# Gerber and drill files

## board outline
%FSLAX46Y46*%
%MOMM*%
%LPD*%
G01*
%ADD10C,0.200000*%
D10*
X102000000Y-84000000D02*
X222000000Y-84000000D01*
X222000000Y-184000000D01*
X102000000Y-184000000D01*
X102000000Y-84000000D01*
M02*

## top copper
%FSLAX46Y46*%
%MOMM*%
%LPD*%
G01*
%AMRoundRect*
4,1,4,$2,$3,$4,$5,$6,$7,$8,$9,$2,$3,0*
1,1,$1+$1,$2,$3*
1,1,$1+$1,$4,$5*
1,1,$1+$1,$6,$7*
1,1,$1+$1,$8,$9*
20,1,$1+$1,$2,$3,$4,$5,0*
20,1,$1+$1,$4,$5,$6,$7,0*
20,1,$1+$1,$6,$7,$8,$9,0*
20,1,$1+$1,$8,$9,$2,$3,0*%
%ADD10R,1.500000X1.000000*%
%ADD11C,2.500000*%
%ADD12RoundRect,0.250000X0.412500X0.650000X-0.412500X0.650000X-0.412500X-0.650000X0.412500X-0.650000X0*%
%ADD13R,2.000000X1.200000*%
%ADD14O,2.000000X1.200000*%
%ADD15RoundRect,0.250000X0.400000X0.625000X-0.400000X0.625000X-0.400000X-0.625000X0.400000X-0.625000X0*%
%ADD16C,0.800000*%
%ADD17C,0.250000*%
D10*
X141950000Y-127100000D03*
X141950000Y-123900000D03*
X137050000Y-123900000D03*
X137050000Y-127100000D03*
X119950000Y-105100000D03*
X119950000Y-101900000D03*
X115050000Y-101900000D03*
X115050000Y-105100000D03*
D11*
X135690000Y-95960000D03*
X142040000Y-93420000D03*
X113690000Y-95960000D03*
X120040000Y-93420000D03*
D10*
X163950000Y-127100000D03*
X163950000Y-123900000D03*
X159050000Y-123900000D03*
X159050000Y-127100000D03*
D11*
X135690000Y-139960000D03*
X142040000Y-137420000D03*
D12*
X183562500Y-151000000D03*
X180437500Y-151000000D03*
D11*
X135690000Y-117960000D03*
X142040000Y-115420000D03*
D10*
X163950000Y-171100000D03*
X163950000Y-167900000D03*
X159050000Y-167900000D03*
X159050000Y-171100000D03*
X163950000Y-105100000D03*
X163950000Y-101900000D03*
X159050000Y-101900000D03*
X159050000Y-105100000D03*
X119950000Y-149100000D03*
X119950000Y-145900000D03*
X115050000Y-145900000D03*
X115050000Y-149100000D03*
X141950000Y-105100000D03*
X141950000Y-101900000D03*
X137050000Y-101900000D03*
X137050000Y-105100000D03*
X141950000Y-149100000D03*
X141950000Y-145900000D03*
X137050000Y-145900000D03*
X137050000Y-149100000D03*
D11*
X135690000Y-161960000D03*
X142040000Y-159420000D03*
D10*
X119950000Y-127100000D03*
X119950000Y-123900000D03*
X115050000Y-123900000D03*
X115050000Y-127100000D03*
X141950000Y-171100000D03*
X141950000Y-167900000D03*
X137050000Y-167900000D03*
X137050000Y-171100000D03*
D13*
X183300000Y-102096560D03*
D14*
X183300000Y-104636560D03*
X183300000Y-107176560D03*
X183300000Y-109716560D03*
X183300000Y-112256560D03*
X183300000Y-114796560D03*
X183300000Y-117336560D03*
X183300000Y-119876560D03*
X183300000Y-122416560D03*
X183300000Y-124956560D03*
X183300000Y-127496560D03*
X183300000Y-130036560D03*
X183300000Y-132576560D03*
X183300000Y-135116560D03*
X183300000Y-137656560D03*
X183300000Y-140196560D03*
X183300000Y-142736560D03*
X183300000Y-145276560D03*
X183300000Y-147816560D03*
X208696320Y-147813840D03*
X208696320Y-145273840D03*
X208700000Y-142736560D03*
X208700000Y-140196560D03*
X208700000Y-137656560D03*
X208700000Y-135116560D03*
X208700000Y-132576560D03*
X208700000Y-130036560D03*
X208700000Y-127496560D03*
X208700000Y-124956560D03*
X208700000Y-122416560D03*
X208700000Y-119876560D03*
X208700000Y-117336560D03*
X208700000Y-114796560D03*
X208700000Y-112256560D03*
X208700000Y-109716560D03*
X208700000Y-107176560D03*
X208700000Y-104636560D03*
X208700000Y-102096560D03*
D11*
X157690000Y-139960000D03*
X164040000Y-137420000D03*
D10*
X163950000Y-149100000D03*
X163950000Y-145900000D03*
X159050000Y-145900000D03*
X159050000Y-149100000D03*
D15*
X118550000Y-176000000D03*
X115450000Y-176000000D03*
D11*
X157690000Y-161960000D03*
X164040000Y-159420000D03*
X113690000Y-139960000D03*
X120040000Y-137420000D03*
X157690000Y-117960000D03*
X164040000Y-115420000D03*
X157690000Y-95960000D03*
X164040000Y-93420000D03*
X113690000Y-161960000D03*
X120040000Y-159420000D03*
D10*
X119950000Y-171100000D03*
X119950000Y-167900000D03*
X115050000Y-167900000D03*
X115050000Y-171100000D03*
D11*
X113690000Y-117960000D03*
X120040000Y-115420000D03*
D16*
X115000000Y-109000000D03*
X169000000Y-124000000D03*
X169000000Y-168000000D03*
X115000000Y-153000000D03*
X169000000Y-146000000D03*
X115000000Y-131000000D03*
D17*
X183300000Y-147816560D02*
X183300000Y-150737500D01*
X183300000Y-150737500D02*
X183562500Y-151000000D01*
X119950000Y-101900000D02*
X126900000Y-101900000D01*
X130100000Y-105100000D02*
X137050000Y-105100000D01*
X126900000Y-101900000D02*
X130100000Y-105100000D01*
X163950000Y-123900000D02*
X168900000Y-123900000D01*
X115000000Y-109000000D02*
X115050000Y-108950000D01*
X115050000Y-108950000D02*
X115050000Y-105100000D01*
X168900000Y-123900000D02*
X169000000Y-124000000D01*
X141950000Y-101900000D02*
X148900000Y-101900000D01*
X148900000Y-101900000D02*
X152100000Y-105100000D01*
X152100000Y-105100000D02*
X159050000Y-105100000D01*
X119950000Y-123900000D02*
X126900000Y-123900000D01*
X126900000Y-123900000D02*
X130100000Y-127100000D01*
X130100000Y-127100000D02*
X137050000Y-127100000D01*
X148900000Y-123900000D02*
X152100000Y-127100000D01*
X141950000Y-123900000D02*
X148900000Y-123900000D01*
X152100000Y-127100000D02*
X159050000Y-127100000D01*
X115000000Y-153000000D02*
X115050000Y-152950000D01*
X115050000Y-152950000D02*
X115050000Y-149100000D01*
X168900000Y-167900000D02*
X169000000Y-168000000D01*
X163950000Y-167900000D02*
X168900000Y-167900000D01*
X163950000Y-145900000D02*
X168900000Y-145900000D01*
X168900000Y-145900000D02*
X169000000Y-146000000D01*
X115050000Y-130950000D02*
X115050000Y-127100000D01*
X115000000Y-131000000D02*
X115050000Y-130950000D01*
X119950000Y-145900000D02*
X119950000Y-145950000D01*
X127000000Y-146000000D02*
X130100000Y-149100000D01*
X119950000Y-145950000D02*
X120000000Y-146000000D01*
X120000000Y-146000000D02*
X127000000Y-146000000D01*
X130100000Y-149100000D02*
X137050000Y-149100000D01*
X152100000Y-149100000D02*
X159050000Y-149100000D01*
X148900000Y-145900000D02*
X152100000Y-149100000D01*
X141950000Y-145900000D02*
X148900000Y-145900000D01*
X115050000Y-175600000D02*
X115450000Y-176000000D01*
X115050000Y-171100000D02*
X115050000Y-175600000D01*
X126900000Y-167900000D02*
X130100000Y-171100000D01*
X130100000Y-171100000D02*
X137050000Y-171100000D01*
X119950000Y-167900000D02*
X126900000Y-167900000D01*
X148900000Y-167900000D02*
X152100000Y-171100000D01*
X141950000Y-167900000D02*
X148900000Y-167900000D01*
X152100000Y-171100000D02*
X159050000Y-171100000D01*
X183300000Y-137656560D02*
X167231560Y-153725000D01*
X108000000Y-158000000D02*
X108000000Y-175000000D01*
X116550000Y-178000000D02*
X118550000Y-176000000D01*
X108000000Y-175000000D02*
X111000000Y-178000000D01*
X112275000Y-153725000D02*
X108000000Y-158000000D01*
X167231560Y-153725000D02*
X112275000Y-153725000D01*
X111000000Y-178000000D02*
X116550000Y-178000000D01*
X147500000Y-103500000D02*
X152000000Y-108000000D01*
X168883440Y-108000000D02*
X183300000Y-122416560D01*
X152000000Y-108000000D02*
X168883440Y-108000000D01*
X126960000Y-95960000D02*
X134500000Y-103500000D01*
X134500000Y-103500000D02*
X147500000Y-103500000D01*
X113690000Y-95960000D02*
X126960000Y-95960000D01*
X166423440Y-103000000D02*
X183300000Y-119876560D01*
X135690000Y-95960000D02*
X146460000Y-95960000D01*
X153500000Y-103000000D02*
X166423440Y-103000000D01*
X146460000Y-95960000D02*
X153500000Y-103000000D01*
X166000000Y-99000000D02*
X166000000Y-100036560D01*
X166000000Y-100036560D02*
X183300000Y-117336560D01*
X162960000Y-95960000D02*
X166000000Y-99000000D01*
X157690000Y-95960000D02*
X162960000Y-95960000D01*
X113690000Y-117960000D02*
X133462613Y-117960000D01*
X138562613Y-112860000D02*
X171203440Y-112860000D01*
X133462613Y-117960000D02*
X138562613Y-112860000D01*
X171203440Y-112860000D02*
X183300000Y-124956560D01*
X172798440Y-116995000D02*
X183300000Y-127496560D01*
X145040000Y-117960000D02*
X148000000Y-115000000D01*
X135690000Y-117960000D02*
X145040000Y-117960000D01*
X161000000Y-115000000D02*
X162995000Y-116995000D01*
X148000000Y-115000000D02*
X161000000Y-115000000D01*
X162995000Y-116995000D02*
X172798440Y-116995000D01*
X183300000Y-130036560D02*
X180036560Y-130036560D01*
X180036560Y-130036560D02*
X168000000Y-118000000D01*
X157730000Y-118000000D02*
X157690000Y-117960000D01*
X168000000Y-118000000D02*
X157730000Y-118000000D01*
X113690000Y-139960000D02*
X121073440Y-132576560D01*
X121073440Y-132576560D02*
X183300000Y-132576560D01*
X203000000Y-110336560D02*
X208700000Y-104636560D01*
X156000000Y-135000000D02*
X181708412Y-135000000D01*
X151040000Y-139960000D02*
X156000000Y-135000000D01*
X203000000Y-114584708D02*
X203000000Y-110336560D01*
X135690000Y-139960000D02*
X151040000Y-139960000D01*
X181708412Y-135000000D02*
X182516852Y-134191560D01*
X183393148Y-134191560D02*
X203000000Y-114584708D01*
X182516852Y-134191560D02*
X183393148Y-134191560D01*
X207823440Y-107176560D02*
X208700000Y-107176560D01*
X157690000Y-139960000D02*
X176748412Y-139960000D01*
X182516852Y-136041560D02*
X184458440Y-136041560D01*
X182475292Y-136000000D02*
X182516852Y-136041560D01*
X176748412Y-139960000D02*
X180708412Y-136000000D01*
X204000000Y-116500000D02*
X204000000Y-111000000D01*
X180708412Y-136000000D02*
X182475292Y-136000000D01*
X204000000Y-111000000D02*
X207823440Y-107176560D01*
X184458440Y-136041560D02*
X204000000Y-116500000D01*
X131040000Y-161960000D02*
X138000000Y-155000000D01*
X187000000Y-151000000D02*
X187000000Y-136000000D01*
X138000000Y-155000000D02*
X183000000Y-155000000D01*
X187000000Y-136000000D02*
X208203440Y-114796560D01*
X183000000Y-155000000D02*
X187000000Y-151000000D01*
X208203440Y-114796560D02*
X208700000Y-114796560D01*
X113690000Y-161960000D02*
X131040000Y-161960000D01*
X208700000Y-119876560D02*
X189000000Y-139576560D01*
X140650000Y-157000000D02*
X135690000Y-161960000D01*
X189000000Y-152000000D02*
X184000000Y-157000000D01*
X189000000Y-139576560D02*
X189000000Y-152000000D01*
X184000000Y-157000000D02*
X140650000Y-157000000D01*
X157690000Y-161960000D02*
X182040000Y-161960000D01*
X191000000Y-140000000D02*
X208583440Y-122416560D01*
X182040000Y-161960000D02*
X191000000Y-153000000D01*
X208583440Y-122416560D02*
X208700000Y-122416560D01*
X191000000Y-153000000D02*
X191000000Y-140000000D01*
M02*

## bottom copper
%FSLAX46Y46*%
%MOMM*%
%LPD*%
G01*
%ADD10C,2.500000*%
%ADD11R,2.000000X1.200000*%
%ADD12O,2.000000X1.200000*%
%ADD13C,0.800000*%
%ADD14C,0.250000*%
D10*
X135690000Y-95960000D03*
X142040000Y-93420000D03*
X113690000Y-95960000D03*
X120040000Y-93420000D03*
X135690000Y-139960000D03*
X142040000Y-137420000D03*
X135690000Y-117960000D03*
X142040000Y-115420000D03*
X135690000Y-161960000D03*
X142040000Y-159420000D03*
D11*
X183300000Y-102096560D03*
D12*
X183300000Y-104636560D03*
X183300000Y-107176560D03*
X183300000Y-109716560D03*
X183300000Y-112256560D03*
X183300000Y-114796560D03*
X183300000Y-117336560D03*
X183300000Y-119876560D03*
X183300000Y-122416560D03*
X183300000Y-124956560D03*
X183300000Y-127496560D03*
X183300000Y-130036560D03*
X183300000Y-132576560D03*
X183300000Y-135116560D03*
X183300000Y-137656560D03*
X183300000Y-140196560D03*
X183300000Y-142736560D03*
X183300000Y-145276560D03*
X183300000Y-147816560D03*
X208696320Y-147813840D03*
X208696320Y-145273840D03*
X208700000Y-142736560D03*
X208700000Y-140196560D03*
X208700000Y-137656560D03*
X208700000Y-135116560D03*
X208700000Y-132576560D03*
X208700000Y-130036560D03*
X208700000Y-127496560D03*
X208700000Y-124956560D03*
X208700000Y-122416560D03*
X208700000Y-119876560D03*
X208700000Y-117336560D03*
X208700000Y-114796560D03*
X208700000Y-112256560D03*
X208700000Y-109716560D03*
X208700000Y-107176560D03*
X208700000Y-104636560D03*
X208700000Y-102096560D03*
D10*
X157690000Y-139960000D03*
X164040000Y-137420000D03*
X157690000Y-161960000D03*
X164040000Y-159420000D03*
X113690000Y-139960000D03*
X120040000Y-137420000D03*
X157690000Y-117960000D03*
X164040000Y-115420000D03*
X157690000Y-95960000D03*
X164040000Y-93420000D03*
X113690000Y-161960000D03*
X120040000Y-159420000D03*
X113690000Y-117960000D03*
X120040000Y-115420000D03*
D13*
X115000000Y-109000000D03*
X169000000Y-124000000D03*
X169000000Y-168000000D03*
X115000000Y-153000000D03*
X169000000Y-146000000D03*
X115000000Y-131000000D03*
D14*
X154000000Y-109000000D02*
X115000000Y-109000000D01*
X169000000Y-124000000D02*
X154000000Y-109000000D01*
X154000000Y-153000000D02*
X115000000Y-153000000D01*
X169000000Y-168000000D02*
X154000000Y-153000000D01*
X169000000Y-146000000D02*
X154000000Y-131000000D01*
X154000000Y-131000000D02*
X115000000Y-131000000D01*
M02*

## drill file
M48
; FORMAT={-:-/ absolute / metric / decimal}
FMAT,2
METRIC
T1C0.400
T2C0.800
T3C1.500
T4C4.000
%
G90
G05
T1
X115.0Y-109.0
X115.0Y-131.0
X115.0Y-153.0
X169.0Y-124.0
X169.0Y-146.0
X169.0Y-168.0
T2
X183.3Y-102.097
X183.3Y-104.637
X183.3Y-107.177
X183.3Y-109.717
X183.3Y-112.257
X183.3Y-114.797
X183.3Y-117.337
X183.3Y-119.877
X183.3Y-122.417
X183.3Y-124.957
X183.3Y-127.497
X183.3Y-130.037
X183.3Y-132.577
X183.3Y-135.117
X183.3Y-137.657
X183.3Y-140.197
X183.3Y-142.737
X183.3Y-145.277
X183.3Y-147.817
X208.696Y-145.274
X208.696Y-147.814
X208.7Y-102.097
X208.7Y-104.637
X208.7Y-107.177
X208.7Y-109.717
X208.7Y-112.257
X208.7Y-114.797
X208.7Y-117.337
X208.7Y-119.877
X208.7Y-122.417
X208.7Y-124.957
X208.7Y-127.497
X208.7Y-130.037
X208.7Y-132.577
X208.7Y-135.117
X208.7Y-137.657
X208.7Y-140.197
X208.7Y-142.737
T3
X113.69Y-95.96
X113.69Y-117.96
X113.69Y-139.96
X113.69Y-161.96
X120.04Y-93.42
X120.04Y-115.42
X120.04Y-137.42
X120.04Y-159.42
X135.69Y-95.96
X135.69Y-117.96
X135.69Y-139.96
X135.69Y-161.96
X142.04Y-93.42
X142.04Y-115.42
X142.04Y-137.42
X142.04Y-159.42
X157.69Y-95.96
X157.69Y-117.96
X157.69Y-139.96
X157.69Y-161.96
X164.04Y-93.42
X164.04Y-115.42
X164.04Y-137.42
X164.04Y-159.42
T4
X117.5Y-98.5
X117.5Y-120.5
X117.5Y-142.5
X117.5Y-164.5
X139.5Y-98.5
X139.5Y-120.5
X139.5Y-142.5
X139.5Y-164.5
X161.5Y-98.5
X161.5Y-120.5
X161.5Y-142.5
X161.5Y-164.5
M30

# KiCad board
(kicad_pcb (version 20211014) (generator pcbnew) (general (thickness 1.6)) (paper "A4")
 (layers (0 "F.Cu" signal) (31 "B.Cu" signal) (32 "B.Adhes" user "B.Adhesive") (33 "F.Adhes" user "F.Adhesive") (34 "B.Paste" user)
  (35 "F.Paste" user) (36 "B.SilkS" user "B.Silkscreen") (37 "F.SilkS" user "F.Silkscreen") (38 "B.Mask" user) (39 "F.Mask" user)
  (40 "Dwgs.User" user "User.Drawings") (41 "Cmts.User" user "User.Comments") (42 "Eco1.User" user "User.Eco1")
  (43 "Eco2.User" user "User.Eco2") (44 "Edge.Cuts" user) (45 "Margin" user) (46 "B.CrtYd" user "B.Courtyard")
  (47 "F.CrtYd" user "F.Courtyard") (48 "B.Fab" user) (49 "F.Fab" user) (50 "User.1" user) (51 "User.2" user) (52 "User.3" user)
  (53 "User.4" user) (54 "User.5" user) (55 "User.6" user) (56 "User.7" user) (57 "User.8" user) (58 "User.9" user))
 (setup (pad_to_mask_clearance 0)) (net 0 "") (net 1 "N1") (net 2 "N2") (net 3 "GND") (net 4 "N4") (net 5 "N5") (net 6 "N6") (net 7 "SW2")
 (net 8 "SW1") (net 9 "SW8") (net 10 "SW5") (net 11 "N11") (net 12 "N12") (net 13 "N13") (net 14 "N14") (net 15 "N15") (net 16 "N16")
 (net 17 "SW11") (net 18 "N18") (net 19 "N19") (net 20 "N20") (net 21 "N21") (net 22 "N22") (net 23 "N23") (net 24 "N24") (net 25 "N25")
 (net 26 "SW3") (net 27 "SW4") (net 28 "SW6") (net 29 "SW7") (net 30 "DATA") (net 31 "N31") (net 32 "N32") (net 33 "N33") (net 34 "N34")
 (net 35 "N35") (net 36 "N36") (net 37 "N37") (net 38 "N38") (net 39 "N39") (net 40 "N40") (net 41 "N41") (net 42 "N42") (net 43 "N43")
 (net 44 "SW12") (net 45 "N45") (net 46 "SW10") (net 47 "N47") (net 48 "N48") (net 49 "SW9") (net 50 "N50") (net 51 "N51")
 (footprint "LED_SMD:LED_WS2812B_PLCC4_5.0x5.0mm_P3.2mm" (layer "F.Cu") (at 139.5 125.5 180)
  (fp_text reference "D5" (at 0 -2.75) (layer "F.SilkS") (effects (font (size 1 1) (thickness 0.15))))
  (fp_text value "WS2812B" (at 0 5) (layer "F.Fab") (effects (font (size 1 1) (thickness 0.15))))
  (pad "1" smd rect (at -2.45 -1.6 180) (size 1.5 1) (layers "F.Cu" "F.Paste" "F.Mask") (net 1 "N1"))
  (pad "2" smd rect (at -2.45 1.6 180) (size 1.5 1) (layers "F.Cu" "F.Paste" "F.Mask") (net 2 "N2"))
  (pad "3" smd rect (at 2.45 1.6 180) (size 1.5 1) (layers "F.Cu" "F.Paste" "F.Mask") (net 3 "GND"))
  (pad "4" smd rect (at 2.45 -1.6 180) (size 1.5 1) (layers "F.Cu" "F.Paste" "F.Mask") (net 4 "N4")))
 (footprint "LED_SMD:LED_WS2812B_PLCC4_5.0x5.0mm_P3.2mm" (layer "F.Cu") (at 117.5 103.5 180)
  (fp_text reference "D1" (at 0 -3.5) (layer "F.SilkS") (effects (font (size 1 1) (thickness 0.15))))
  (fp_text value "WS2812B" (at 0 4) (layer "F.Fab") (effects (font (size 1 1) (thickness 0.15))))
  (pad "1" smd rect (at -2.45 -1.6 180) (size 1.5 1) (layers "F.Cu" "F.Paste" "F.Mask") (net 1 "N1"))
  (pad "2" smd rect (at -2.45 1.6 180) (size 1.5 1) (layers "F.Cu" "F.Paste" "F.Mask") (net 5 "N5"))
  (pad "3" smd rect (at 2.45 1.6 180) (size 1.5 1) (layers "F.Cu" "F.Paste" "F.Mask") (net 3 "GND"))
  (pad "4" smd rect (at 2.45 -1.6 180) (size 1.5 1) (layers "F.Cu" "F.Paste" "F.Mask") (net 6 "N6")))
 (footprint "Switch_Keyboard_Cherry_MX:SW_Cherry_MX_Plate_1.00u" (layer "F.Cu") (at 139.5 98.5)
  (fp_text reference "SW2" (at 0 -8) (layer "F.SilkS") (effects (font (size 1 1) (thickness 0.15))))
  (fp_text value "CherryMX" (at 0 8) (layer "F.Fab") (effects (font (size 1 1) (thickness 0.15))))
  (pad "" np_thru_hole circle locked (at 0 0) (size 4 4) (drill 4) (layers *.Cu *.Mask))
  (pad "" smd circle locked (at -3.81 -2.54) (size 1.55 1.55) (layers "F.Mask"))
  (pad "" smd circle locked (at 2.54 -5.08) (size 1.55 1.55) (layers "F.Mask"))
  (pad "1" thru_hole circle locked (at -3.81 -2.54) (size 2.5 2.5) (drill 1.5) (layers *.Cu "B.Mask") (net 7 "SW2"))
  (pad "2" thru_hole circle locked (at 2.54 -5.08) (size 2.5 2.5) (drill 1.5) (layers *.Cu "B.Mask") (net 3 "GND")))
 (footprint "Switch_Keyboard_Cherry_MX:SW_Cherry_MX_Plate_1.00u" (layer "F.Cu") (at 117.5 98.5)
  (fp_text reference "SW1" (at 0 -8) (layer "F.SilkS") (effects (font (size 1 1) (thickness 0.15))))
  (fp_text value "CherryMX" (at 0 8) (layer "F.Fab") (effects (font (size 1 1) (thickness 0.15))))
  (pad "" smd circle locked (at -3.81 -2.54) (size 1.55 1.55) (layers "F.Mask"))
  (pad "" smd circle locked (at 2.54 -5.08) (size 1.55 1.55) (layers "F.Mask"))
  (pad "" np_thru_hole circle locked (at 0 0) (size 4 4) (drill 4) (layers *.Cu *.Mask))
  (pad "1" thru_hole circle locked (at -3.81 -2.54) (size 2.5 2.5) (drill 1.5) (layers *.Cu "B.Mask") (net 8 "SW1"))
  (pad "2" thru_hole circle locked (at 2.54 -5.08) (size 2.5 2.5) (drill 1.5) (layers *.Cu "B.Mask") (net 3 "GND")))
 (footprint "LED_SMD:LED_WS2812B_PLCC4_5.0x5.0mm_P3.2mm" (layer "F.Cu") (at 161.5 125.5 180)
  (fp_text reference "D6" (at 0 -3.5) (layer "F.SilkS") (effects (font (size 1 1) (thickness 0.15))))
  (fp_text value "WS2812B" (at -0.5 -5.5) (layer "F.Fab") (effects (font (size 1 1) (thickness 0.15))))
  (pad "1" smd rect (at -2.45 -1.6 180) (size 1.5 1) (layers "F.Cu" "F.Paste" "F.Mask") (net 1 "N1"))
  (pad "2" smd rect (at -2.45 1.6 180) (size 1.5 1) (layers "F.Cu" "F.Paste" "F.Mask") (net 6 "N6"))
  (pad "3" smd rect (at 2.45 1.6 180) (size 1.5 1) (layers "F.Cu" "F.Paste" "F.Mask") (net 3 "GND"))
  (pad "4" smd rect (at 2.45 -1.6 180) (size 1.5 1) (layers "F.Cu" "F.Paste" "F.Mask") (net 2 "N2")))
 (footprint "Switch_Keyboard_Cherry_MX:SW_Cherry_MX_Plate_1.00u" (layer "F.Cu") (at 139.5 142.5)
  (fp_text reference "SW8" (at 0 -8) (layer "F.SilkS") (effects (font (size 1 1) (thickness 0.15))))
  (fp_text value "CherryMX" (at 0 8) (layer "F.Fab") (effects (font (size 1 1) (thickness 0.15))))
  (pad "" smd circle locked (at 2.54 -5.08) (size 1.55 1.55) (layers "F.Mask"))
  (pad "" np_thru_hole circle locked (at 0 0) (size 4 4) (drill 4) (layers *.Cu *.Mask))
  (pad "" smd circle locked (at -3.81 -2.54) (size 1.55 1.55) (layers "F.Mask"))
  (pad "1" thru_hole circle locked (at -3.81 -2.54) (size 2.5 2.5) (drill 1.5) (layers *.Cu "B.Mask") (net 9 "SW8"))
  (pad "2" thru_hole circle locked (at 2.54 -5.08) (size 2.5 2.5) (drill 1.5) (layers *.Cu "B.Mask") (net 3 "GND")))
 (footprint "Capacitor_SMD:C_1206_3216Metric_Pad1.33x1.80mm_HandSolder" (layer "F.Cu") (at 182 151 180)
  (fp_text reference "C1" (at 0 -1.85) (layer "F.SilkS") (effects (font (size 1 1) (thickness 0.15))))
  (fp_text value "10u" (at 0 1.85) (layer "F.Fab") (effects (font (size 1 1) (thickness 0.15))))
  (pad "1" smd roundrect (at -1.5625 0 180) (size 1.325 1.8) (layers "F.Cu" "F.Paste" "F.Mask") (roundrect_rratio 0.188679) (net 1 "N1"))
  (pad "2" smd roundrect (at 1.5625 0 180) (size 1.325 1.8) (layers "F.Cu" "F.Paste" "F.Mask") (roundrect_rratio 0.188679) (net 3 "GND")))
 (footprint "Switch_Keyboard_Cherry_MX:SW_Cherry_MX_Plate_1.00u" (layer "F.Cu") (at 139.5 120.5)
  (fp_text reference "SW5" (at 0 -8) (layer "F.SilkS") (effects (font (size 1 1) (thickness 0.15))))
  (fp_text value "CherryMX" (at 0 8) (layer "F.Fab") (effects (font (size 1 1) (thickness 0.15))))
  (pad "" np_thru_hole circle locked (at 0 0) (size 4 4) (drill 4) (layers *.Cu *.Mask))
  (pad "" smd circle locked (at 2.54 -5.08) (size 1.55 1.55) (layers "F.Mask"))
  (pad "" smd circle locked (at -3.81 -2.54) (size 1.55 1.55) (layers "F.Mask"))
  (pad "1" thru_hole circle locked (at -3.81 -2.54) (size 2.5 2.5) (drill 1.5) (layers *.Cu "B.Mask") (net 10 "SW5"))
  (pad "2" thru_hole circle locked (at 2.54 -5.08) (size 2.5 2.5) (drill 1.5) (layers *.Cu "B.Mask") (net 3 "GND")))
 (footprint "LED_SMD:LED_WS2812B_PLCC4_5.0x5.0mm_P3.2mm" (layer "F.Cu") (at 161.5 169.5 180)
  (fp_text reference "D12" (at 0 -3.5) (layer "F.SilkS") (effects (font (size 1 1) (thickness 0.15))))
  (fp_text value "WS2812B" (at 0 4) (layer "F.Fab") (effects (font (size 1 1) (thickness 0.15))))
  (pad "1" smd rect (at -2.45 -1.6 180) (size 1.5 1) (layers "F.Cu" "F.Paste" "F.Mask") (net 1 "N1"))
  (pad "2" smd rect (at -2.45 1.6 180) (size 1.5 1) (layers "F.Cu" "F.Paste" "F.Mask") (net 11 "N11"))
  (pad "3" smd rect (at 2.45 1.6 180) (size 1.5 1) (layers "F.Cu" "F.Paste" "F.Mask") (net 3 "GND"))
  (pad "4" smd rect (at 2.45 -1.6 180) (size 1.5 1) (layers "F.Cu" "F.Paste" "F.Mask") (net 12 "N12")))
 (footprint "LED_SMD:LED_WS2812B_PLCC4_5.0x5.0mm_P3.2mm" (layer "F.Cu") (at 161.5 103.5 180)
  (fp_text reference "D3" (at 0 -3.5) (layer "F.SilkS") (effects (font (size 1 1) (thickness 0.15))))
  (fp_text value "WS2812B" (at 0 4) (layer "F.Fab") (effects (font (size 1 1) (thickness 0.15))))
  (pad "1" smd rect (at -2.45 -1.6 180) (size 1.5 1) (layers "F.Cu" "F.Paste" "F.Mask") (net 1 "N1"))
  (pad "2" smd rect (at -2.45 1.6 180) (size 1.5 1) (layers "F.Cu" "F.Paste" "F.Mask") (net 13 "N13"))
  (pad "3" smd rect (at 2.45 1.6 180) (size 1.5 1) (layers "F.Cu" "F.Paste" "F.Mask") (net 3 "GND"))
  (pad "4" smd rect (at 2.45 -1.6 180) (size 1.5 1) (layers "F.Cu" "F.Paste" "F.Mask") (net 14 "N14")))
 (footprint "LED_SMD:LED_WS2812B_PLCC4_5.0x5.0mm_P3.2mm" (layer "F.Cu") (at 117.5 147.5 180)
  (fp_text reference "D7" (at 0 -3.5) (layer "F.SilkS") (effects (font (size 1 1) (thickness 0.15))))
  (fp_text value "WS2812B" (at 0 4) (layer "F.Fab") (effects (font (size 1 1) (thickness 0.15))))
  (pad "1" smd rect (at -2.45 -1.6 180) (size 1.5 1) (layers "F.Cu" "F.Paste" "F.Mask") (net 1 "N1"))
  (pad "2" smd rect (at -2.45 1.6 180) (size 1.5 1) (layers "F.Cu" "F.Paste" "F.Mask") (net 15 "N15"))
  (pad "3" smd rect (at 2.45 1.6 180) (size 1.5 1) (layers "F.Cu" "F.Paste" "F.Mask") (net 3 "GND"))
  (pad "4" smd rect (at 2.45 -1.6 180) (size 1.5 1) (layers "F.Cu" "F.Paste" "F.Mask") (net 11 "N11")))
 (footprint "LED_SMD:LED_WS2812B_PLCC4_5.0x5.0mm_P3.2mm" (layer "F.Cu") (at 139.5 103.5 180)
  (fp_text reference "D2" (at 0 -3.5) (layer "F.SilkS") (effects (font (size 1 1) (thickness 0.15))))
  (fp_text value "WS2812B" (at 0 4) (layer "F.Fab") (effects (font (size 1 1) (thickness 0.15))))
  (pad "1" smd rect (at -2.45 -1.6 180) (size 1.5 1) (layers "F.Cu" "F.Paste" "F.Mask") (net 1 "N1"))
  (pad "2" smd rect (at -2.45 1.6 180) (size 1.5 1) (layers "F.Cu" "F.Paste" "F.Mask") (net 14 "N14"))
  (pad "3" smd rect (at 2.45 1.6 180) (size 1.5 1) (layers "F.Cu" "F.Paste" "F.Mask") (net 3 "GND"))
  (pad "4" smd rect (at 2.45 -1.6 180) (size 1.5 1) (layers "F.Cu" "F.Paste" "F.Mask") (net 5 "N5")))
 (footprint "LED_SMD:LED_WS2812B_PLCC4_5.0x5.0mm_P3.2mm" (layer "F.Cu") (at 139.5 147.5 180)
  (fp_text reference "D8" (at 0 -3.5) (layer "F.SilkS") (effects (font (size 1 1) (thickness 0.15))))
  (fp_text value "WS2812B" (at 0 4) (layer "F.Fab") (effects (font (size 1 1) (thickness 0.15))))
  (pad "1" smd rect (at -2.45 -1.6 180) (size 1.5 1) (layers "F.Cu" "F.Paste" "F.Mask") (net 1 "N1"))
  (pad "2" smd rect (at -2.45 1.6 180) (size 1.5 1) (layers "F.Cu" "F.Paste" "F.Mask") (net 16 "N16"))
  (pad "3" smd rect (at 2.45 1.6 180) (size 1.5 1) (layers "F.Cu" "F.Paste" "F.Mask") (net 3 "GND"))
  (pad "4" smd rect (at 2.45 -1.6 180) (size 1.5 1) (layers "F.Cu" "F.Paste" "F.Mask") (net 15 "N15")))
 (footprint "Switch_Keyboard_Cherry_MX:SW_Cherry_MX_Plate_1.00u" (layer "F.Cu") (at 139.5 164.5)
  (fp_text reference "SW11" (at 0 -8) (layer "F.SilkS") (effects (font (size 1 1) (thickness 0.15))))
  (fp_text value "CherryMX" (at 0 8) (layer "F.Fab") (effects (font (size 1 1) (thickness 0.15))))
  (pad "" np_thru_hole circle locked (at 0 0) (size 4 4) (drill 4) (layers *.Cu *.Mask))
  (pad "" smd circle locked (at 2.54 -5.08) (size 1.55 1.55) (layers "F.Mask"))
  (pad "" smd circle locked (at -3.81 -2.54) (size 1.55 1.55) (layers "F.Mask"))
  (pad "1" thru_hole circle locked (at -3.81 -2.54) (size 2.5 2.5) (drill 1.5) (layers *.Cu "B.Mask") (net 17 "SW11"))
  (pad "2" thru_hole circle locked (at 2.54 -5.08) (size 2.5 2.5) (drill 1.5) (layers *.Cu "B.Mask") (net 3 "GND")))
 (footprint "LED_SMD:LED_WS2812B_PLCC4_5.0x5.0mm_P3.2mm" (layer "F.Cu") (at 117.5 125.5 180)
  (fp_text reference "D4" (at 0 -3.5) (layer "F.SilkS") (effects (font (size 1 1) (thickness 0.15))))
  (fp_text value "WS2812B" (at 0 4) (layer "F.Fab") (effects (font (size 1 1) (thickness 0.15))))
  (pad "1" smd rect (at -2.45 -1.6 180) (size 1.5 1) (layers "F.Cu" "F.Paste" "F.Mask") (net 1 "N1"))
  (pad "2" smd rect (at -2.45 1.6 180) (size 1.5 1) (layers "F.Cu" "F.Paste" "F.Mask") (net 4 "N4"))
  (pad "3" smd rect (at 2.45 1.6 180) (size 1.5 1) (layers "F.Cu" "F.Paste" "F.Mask") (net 3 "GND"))
  (pad "4" smd rect (at 2.45 -1.6 180) (size 1.5 1) (layers "F.Cu" "F.Paste" "F.Mask") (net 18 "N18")))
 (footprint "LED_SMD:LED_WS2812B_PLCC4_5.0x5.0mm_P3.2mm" (layer "F.Cu") (at 139.5 169.5 180)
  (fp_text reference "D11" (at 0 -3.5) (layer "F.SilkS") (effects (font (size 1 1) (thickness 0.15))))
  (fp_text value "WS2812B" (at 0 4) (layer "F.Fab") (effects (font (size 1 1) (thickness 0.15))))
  (pad "1" smd rect (at -2.45 -1.6 180) (size 1.5 1) (layers "F.Cu" "F.Paste" "F.Mask") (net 1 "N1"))
  (pad "2" smd rect (at -2.45 1.6 180) (size 1.5 1) (layers "F.Cu" "F.Paste" "F.Mask") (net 12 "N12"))
  (pad "3" smd rect (at 2.45 1.6 180) (size 1.5 1) (layers "F.Cu" "F.Paste" "F.Mask") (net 3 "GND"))
  (pad "4" smd rect (at 2.45 -1.6 180) (size 1.5 1) (layers "F.Cu" "F.Paste" "F.Mask") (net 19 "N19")))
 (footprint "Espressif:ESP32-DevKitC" (layer "F.Cu") (at 183.3 102.09656)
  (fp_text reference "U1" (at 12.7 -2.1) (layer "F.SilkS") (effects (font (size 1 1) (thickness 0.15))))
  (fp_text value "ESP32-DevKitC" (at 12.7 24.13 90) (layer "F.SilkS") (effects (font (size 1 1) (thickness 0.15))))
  (pad "1" thru_hole rect (at 0 0 270) (size 1.2 2) (drill 0.8) (layers *.Cu *.Mask) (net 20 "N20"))
  (pad "2" thru_hole oval (at 0 2.54 270) (size 1.2 2) (drill 0.8) (layers *.Cu *.Mask) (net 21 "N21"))
  (pad "3" thru_hole oval (at 0 5.08 270) (size 1.2 2) (drill 0.8) (layers *.Cu *.Mask) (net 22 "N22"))
  (pad "4" thru_hole oval (at 0 7.62 270) (size 1.2 2) (drill 0.8) (layers *.Cu *.Mask) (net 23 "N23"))
  (pad "5" thru_hole oval (at 0 10.16 270) (size 1.2 2) (drill 0.8) (layers *.Cu *.Mask) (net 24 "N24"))
  (pad "6" thru_hole oval (at 0 12.7 270) (size 1.2 2) (drill 0.8) (layers *.Cu *.Mask) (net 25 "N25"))
  (pad "7" thru_hole oval (at 0 15.24 270) (size 1.2 2) (drill 0.8) (layers *.Cu *.Mask) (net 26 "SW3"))
  (pad "8" thru_hole oval (at 0 17.78 270) (size 1.2 2) (drill 0.8) (layers *.Cu *.Mask) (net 7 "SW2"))
  (pad "9" thru_hole oval (at 0 20.32 270) (size 1.2 2) (drill 0.8) (layers *.Cu *.Mask) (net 8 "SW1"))
  (pad "10" thru_hole oval (at 0 22.86 270) (size 1.2 2) (drill 0.8) (layers *.Cu *.Mask) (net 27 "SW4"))
  (pad "11" thru_hole oval (at 0 25.4 270) (size 1.2 2) (drill 0.8) (layers *.Cu *.Mask) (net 10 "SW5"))
  (pad "12" thru_hole oval (at 0 27.94 270) (size 1.2 2) (drill 0.8) (layers *.Cu *.Mask) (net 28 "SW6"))
  (pad "13" thru_hole oval (at 0 30.48 270) (size 1.2 2) (drill 0.8) (layers *.Cu *.Mask) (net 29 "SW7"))
  (pad "14" thru_hole oval (at 0 33.02 270) (size 1.2 2) (drill 0.8) (layers *.Cu *.Mask) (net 3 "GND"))
  (pad "15" thru_hole oval (at 0 35.56 270) (size 1.2 2) (drill 0.8) (layers *.Cu *.Mask) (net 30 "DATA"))
  (pad "16" thru_hole oval (at 0 38.1 270) (size 1.2 2) (drill 0.8) (layers *.Cu *.Mask) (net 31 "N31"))
  (pad "17" thru_hole oval (at 0 40.64 270) (size 1.2 2) (drill 0.8) (layers *.Cu *.Mask) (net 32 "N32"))
  (pad "18" thru_hole oval (at 0 43.18 270) (size 1.2 2) (drill 0.8) (layers *.Cu *.Mask) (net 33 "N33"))
  (pad "19" thru_hole oval (at 0 45.72 270) (size 1.2 2) (drill 0.8) (layers *.Cu *.Mask) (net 1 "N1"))
  (pad "20" thru_hole oval (at 25.39632 45.71728 270) (size 1.2 2) (drill 0.8) (layers *.Cu *.Mask) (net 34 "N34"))
  (pad "21" thru_hole oval (at 25.39632 43.17728 270) (size 1.2 2) (drill 0.8) (layers *.Cu *.Mask) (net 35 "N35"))
  (pad "22" thru_hole oval (at 25.4 40.64 270) (size 1.2 2) (drill 0.8) (layers *.Cu *.Mask) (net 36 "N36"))
  (pad "23" thru_hole oval (at 25.4 38.1 270) (size 1.2 2) (drill 0.8) (layers *.Cu *.Mask) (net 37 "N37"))
  (pad "24" thru_hole oval (at 25.4 35.56 270) (size 1.2 2) (drill 0.8) (layers *.Cu *.Mask) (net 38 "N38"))
  (pad "25" thru_hole oval (at 25.4 33.02 270) (size 1.2 2) (drill 0.8) (layers *.Cu *.Mask) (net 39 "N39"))
  (pad "26" thru_hole oval (at 25.4 30.48 270) (size 1.2 2) (drill 0.8) (layers *.Cu *.Mask) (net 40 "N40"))
  (pad "27" thru_hole oval (at 25.4 27.94 270) (size 1.2 2) (drill 0.8) (layers *.Cu *.Mask) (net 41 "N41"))
  (pad "28" thru_hole oval (at 25.4 25.4 270) (size 1.2 2) (drill 0.8) (layers *.Cu *.Mask) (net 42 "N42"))
  (pad "29" thru_hole oval (at 25.4 22.86 270) (size 1.2 2) (drill 0.8) (layers *.Cu *.Mask) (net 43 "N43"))
  (pad "30" thru_hole oval (at 25.4 20.32 270) (size 1.2 2) (drill 0.8) (layers *.Cu *.Mask) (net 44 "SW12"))
  (pad "31" thru_hole oval (at 25.4 17.78 270) (size 1.2 2) (drill 0.8) (layers *.Cu *.Mask) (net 17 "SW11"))
  (pad "32" thru_hole oval (at 25.4 15.24 270) (size 1.2 2) (drill 0.8) (layers *.Cu *.Mask) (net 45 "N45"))
  (pad "33" thru_hole oval (at 25.4 12.7 270) (size 1.2 2) (drill 0.8) (layers *.Cu *.Mask) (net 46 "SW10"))
  (pad "34" thru_hole oval (at 25.4 10.16 270) (size 1.2 2) (drill 0.8) (layers *.Cu *.Mask) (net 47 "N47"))
  (pad "35" thru_hole oval (at 25.4 7.62 270) (size 1.2 2) (drill 0.8) (layers *.Cu *.Mask) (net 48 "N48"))
  (pad "36" thru_hole oval (at 25.4 5.08 270) (size 1.2 2) (drill 0.8) (layers *.Cu *.Mask) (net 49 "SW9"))
  (pad "37" thru_hole oval (at 25.4 2.54 270) (size 1.2 2) (drill 0.8) (layers *.Cu *.Mask) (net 9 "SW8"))
  (pad "38" thru_hole oval (at 25.4 0 270) (size 1.2 2) (drill 0.8) (layers *.Cu *.Mask) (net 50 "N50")))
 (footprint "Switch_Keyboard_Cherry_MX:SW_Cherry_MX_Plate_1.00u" (layer "F.Cu") (at 161.5 142.5)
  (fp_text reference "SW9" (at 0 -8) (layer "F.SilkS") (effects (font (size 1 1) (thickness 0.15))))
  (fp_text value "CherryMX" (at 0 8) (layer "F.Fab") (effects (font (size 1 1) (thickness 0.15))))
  (pad "" smd circle locked (at -3.81 -2.54) (size 1.55 1.55) (layers "F.Mask"))
  (pad "" np_thru_hole circle locked (at 0 0) (size 4 4) (drill 4) (layers *.Cu *.Mask))
  (pad "" smd circle locked (at 2.54 -5.08) (size 1.55 1.55) (layers "F.Mask"))
  (pad "1" thru_hole circle locked (at -3.81 -2.54) (size 2.5 2.5) (drill 1.5) (layers *.Cu "B.Mask") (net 49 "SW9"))
  (pad "2" thru_hole circle locked (at 2.54 -5.08) (size 2.5 2.5) (drill 1.5) (layers *.Cu "B.Mask") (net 3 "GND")))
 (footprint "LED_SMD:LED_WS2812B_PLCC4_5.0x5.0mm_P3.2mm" (layer "F.Cu") (at 161.5 147.5 180)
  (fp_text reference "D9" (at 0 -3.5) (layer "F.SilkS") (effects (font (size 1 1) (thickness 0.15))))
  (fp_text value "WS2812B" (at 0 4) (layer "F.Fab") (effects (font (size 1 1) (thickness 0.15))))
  (pad "1" smd rect (at -2.45 -1.6 180) (size 1.5 1) (layers "F.Cu" "F.Paste" "F.Mask") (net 1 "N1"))
  (pad "2" smd rect (at -2.45 1.6 180) (size 1.5 1) (layers "F.Cu" "F.Paste" "F.Mask") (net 18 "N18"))
  (pad "3" smd rect (at 2.45 1.6 180) (size 1.5 1) (layers "F.Cu" "F.Paste" "F.Mask") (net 3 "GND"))
  (pad "4" smd rect (at 2.45 -1.6 180) (size 1.5 1) (layers "F.Cu" "F.Paste" "F.Mask") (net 16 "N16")))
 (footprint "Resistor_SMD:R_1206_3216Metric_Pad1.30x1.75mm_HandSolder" (layer "F.Cu") (at 117 176 180)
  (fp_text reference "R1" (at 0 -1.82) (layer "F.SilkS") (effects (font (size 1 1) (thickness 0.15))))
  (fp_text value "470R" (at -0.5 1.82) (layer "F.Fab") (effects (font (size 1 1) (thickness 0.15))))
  (pad "1" smd roundrect (at -1.55 0 180) (size 1.3 1.75) (layers "F.Cu" "F.Paste" "F.Mask") (roundrect_rratio 0.192308) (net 30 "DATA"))
  (pad "2" smd roundrect (at 1.55 0 180) (size 1.3 1.75) (layers "F.Cu" "F.Paste" "F.Mask") (roundrect_rratio 0.192308) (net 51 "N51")))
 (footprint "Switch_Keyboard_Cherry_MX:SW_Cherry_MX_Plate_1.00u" (layer "F.Cu") (at 161.5 164.5)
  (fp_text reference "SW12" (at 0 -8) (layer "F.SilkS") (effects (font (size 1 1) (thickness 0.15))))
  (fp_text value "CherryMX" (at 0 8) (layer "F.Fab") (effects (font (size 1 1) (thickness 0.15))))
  (pad "" smd circle locked (at 2.54 -5.08) (size 1.55 1.55) (layers "F.Mask"))
  (pad "" smd circle locked (at -3.81 -2.54) (size 1.55 1.55) (layers "F.Mask"))
  (pad "" np_thru_hole circle locked (at 0 0) (size 4 4) (drill 4) (layers *.Cu *.Mask))
  (pad "1" thru_hole circle locked (at -3.81 -2.54) (size 2.5 2.5) (drill 1.5) (layers *.Cu "B.Mask") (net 44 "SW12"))
  (pad "2" thru_hole circle locked (at 2.54 -5.08) (size 2.5 2.5) (drill 1.5) (layers *.Cu "B.Mask") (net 3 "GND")))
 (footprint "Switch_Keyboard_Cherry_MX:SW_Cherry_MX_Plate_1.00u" (layer "F.Cu") (at 117.5 142.5)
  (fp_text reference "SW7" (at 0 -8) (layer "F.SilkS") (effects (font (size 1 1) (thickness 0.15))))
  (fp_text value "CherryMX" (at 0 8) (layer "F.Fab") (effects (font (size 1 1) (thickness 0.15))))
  (pad "" smd circle locked (at 2.54 -5.08) (size 1.55 1.55) (layers "F.Mask"))
  (pad "" smd circle locked (at -3.81 -2.54) (size 1.55 1.55) (layers "F.Mask"))
  (pad "" np_thru_hole circle locked (at 0 0) (size 4 4) (drill 4) (layers *.Cu *.Mask))
  (pad "1" thru_hole circle locked (at -3.81 -2.54) (size 2.5 2.5) (drill 1.5) (layers *.Cu "B.Mask") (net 29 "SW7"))
  (pad "2" thru_hole circle locked (at 2.54 -5.08) (size 2.5 2.5) (drill 1.5) (layers *.Cu "B.Mask") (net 3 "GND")))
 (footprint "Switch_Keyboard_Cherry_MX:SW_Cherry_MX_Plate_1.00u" (layer "F.Cu") (at 161.5 120.5)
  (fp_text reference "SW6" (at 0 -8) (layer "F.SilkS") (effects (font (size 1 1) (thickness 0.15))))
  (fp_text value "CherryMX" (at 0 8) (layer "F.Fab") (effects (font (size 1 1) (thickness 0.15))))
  (pad "" np_thru_hole circle locked (at 0 0) (size 4 4) (drill 4) (layers *.Cu *.Mask))
  (pad "" smd circle locked (at 2.54 -5.08) (size 1.55 1.55) (layers "F.Mask"))
  (pad "" smd circle locked (at -3.81 -2.54) (size 1.55 1.55) (layers "F.Mask"))
  (pad "1" thru_hole circle locked (at -3.81 -2.54) (size 2.5 2.5) (drill 1.5) (layers *.Cu "B.Mask") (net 28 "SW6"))
  (pad "2" thru_hole circle locked (at 2.54 -5.08) (size 2.5 2.5) (drill 1.5) (layers *.Cu "B.Mask") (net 3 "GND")))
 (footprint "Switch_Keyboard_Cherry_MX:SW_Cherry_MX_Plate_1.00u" (layer "F.Cu") (at 161.5 98.5)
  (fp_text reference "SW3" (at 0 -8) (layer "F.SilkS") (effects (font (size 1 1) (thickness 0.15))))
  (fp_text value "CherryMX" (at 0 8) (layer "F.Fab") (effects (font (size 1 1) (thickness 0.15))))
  (pad "" np_thru_hole circle locked (at 0 0) (size 4 4) (drill 4) (layers *.Cu *.Mask))
  (pad "" smd circle locked (at -3.81 -2.54) (size 1.55 1.55) (layers "F.Mask"))
  (pad "" smd circle locked (at 2.54 -5.08) (size 1.55 1.55) (layers "F.Mask"))
  (pad "1" thru_hole circle locked (at -3.81 -2.54) (size 2.5 2.5) (drill 1.5) (layers *.Cu "B.Mask") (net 26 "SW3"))
  (pad "2" thru_hole circle locked (at 2.54 -5.08) (size 2.5 2.5) (drill 1.5) (layers *.Cu "B.Mask") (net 3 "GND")))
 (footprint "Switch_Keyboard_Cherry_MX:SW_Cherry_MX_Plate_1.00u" (layer "F.Cu") (at 117.5 164.5)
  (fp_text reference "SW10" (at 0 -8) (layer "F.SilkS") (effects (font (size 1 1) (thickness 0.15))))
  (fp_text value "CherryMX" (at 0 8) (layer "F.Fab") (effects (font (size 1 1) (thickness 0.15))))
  (pad "" smd circle locked (at -3.81 -2.54) (size 1.55 1.55) (layers "F.Mask"))
  (pad "" np_thru_hole circle locked (at 0 0) (size 4 4) (drill 4) (layers *.Cu *.Mask))
  (pad "" smd circle locked (at 2.54 -5.08) (size 1.55 1.55) (layers "F.Mask"))
  (pad "1" thru_hole circle locked (at -3.81 -2.54) (size 2.5 2.5) (drill 1.5) (layers *.Cu "B.Mask") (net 46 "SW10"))
  (pad "2" thru_hole circle locked (at 2.54 -5.08) (size 2.5 2.5) (drill 1.5) (layers *.Cu "B.Mask") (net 3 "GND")))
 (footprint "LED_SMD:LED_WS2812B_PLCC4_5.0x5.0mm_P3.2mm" (layer "F.Cu") (at 117.5 169.5 180)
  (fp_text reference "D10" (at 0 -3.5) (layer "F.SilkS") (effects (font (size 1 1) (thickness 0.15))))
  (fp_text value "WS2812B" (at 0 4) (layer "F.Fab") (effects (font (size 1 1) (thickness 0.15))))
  (pad "1" smd rect (at -2.45 -1.6 180) (size 1.5 1) (layers "F.Cu" "F.Paste" "F.Mask") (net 1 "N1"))
  (pad "2" smd rect (at -2.45 1.6 180) (size 1.5 1) (layers "F.Cu" "F.Paste" "F.Mask") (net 19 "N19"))
  (pad "3" smd rect (at 2.45 1.6 180) (size 1.5 1) (layers "F.Cu" "F.Paste" "F.Mask") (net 3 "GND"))
  (pad "4" smd rect (at 2.45 -1.6 180) (size 1.5 1) (layers "F.Cu" "F.Paste" "F.Mask") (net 51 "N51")))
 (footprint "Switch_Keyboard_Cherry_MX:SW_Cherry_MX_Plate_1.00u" (layer "F.Cu") (at 117.5 120.5)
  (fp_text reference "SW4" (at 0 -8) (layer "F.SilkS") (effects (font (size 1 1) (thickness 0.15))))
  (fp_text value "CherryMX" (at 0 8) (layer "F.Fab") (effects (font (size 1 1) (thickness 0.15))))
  (pad "" smd circle locked (at -3.81 -2.54) (size 1.55 1.55) (layers "F.Mask"))
  (pad "" np_thru_hole circle locked (at 0 0) (size 4 4) (drill 4) (layers *.Cu *.Mask))
  (pad "" smd circle locked (at 2.54 -5.08) (size 1.55 1.55) (layers "F.Mask"))
  (pad "1" thru_hole circle locked (at -3.81 -2.54) (size 2.5 2.5) (drill 1.5) (layers *.Cu "B.Mask") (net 27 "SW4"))
  (pad "2" thru_hole circle locked (at 2.54 -5.08) (size 2.5 2.5) (drill 1.5) (layers *.Cu "B.Mask") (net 3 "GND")))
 (gr_rect (start 102 84) (end 222 184) (layer "Edge.Cuts") (width 0.2) (fill none))
 (segment (start 183.3 147.81656) (end 183.3 150.7375) (width 0.25) (layer "F.Cu") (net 1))
 (segment (start 183.3 150.7375) (end 183.5625 151) (width 0.25) (layer "F.Cu") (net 1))
 (segment (start 119.95 101.9) (end 126.9 101.9) (width 0.25) (layer "F.Cu") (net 5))
 (segment (start 130.1 105.1) (end 137.05 105.1) (width 0.25) (layer "F.Cu") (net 5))
 (segment (start 126.9 101.9) (end 130.1 105.1) (width 0.25) (layer "F.Cu") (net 5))
 (segment (start 163.95 123.9) (end 168.9 123.9) (width 0.25) (layer "F.Cu") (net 6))
 (segment (start 115 109) (end 115.05 108.95) (width 0.25) (layer "F.Cu") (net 6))
 (segment (start 115.05 108.95) (end 115.05 105.1) (width 0.25) (layer "F.Cu") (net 6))
 (segment (start 168.9 123.9) (end 169 124) (width 0.25) (layer "F.Cu") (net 6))
 (via (at 115 109) (size 0.8) (drill 0.4) (layers "F.Cu" "B.Cu") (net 6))
 (via (at 169 124) (size 0.8) (drill 0.4) (layers "F.Cu" "B.Cu") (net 6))
 (segment (start 154 109) (end 115 109) (width 0.25) (layer "B.Cu") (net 6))
 (segment (start 169 124) (end 154 109) (width 0.25) (layer "B.Cu") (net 6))
 (segment (start 141.95 101.9) (end 148.9 101.9) (width 0.25) (layer "F.Cu") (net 14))
 (segment (start 148.9 101.9) (end 152.1 105.1) (width 0.25) (layer "F.Cu") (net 14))
 (segment (start 152.1 105.1) (end 159.05 105.1) (width 0.25) (layer "F.Cu") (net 14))
 (segment (start 119.95 123.9) (end 126.9 123.9) (width 0.25) (layer "F.Cu") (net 4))
 (segment (start 126.9 123.9) (end 130.1 127.1) (width 0.25) (layer "F.Cu") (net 4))
 (segment (start 130.1 127.1) (end 137.05 127.1) (width 0.25) (layer "F.Cu") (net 4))
 (segment (start 148.9 123.9) (end 152.1 127.1) (width 0.25) (layer "F.Cu") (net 2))
 (segment (start 141.95 123.9) (end 148.9 123.9) (width 0.25) (layer "F.Cu") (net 2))
 (segment (start 152.1 127.1) (end 159.05 127.1) (width 0.25) (layer "F.Cu") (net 2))
 (segment (start 115 153) (end 115.05 152.95) (width 0.25) (layer "F.Cu") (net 11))
 (segment (start 115.05 152.95) (end 115.05 149.1) (width 0.25) (layer "F.Cu") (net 11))
 (segment (start 168.9 167.9) (end 169 168) (width 0.25) (layer "F.Cu") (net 11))
 (segment (start 163.95 167.9) (end 168.9 167.9) (width 0.25) (layer "F.Cu") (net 11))
 (via (at 169 168) (size 0.8) (drill 0.4) (layers "F.Cu" "B.Cu") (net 11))
 (via (at 115 153) (size 0.8) (drill 0.4) (layers "F.Cu" "B.Cu") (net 11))
 (segment (start 154 153) (end 115 153) (width 0.25) (layer "B.Cu") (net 11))
 (segment (start 169 168) (end 154 153) (width 0.25) (layer "B.Cu") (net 11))
 (segment (start 163.95 145.9) (end 168.9 145.9) (width 0.25) (layer "F.Cu") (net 18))
 (segment (start 168.9 145.9) (end 169 146) (width 0.25) (layer "F.Cu") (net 18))
 (segment (start 115.05 130.95) (end 115.05 127.1) (width 0.25) (layer "F.Cu") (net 18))
 (segment (start 115 131) (end 115.05 130.95) (width 0.25) (layer "F.Cu") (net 18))
 (via (at 169 146) (size 0.8) (drill 0.4) (layers "F.Cu" "B.Cu") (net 18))
 (via (at 115 131) (size 0.8) (drill 0.4) (layers "F.Cu" "B.Cu") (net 18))
 (segment (start 169 146) (end 154 131) (width 0.25) (layer "B.Cu") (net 18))
 (segment (start 154 131) (end 115 131) (width 0.25) (layer "B.Cu") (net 18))
 (segment (start 119.95 145.9) (end 119.95 145.95) (width 0.25) (layer "F.Cu") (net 15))
 (segment (start 127 146) (end 130.1 149.1) (width 0.25) (layer "F.Cu") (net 15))
 (segment (start 119.95 145.95) (end 120 146) (width 0.25) (layer "F.Cu") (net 15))
 (segment (start 120 146) (end 127 146) (width 0.25) (layer "F.Cu") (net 15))
 (segment (start 130.1 149.1) (end 137.05 149.1) (width 0.25) (layer "F.Cu") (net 15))
 (segment (start 152.1 149.1) (end 159.05 149.1) (width 0.25) (layer "F.Cu") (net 16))
 (segment (start 148.9 145.9) (end 152.1 149.1) (width 0.25) (layer "F.Cu") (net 16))
 (segment (start 141.95 145.9) (end 148.9 145.9) (width 0.25) (layer "F.Cu") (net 16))
 (segment (start 115.05 175.6) (end 115.45 176) (width 0.25) (layer "F.Cu") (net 51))
 (segment (start 115.05 171.1) (end 115.05 175.6) (width 0.25) (layer "F.Cu") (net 51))
 (segment (start 126.9 167.9) (end 130.1 171.1) (width 0.25) (layer "F.Cu") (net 19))
 (segment (start 130.1 171.1) (end 137.05 171.1) (width 0.25) (layer "F.Cu") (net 19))
 (segment (start 119.95 167.9) (end 126.9 167.9) (width 0.25) (layer "F.Cu") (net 19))
 (segment (start 148.9 167.9) (end 152.1 171.1) (width 0.25) (layer "F.Cu") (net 12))
 (segment (start 141.95 167.9) (end 148.9 167.9) (width 0.25) (layer "F.Cu") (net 12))
 (segment (start 152.1 171.1) (end 159.05 171.1) (width 0.25) (layer "F.Cu") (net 12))
 (segment (start 183.3 137.65656) (end 167.23156 153.725) (width 0.25) (layer "F.Cu") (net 30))
 (segment (start 108 158) (end 108 175) (width 0.25) (layer "F.Cu") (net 30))
 (segment (start 116.55 178) (end 118.55 176) (width 0.25) (layer "F.Cu") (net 30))
 (segment (start 108 175) (end 111 178) (width 0.25) (layer "F.Cu") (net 30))
 (segment (start 112.275 153.725) (end 108 158) (width 0.25) (layer "F.Cu") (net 30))
 (segment (start 167.23156 153.725) (end 112.275 153.725) (width 0.25) (layer "F.Cu") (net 30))
 (segment (start 111 178) (end 116.55 178) (width 0.25) (layer "F.Cu") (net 30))
 (segment (start 147.5 103.5) (end 152 108) (width 0.25) (layer "F.Cu") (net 8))
 (segment (start 168.88344 108) (end 183.3 122.41656) (width 0.25) (layer "F.Cu") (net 8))
 (segment (start 152 108) (end 168.88344 108) (width 0.25) (layer "F.Cu") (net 8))
 (segment (start 126.96 95.96) (end 134.5 103.5) (width 0.25) (layer "F.Cu") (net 8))
 (segment (start 134.5 103.5) (end 147.5 103.5) (width 0.25) (layer "F.Cu") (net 8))
 (segment (start 113.69 95.96) (end 126.96 95.96) (width 0.25) (layer "F.Cu") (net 8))
 (segment (start 166.42344 103) (end 183.3 119.87656) (width 0.25) (layer "F.Cu") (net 7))
 (segment (start 135.69 95.96) (end 146.46 95.96) (width 0.25) (layer "F.Cu") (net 7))
 (segment (start 153.5 103) (end 166.42344 103) (width 0.25) (layer "F.Cu") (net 7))
 (segment (start 146.46 95.96) (end 153.5 103) (width 0.25) (layer "F.Cu") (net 7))
 (segment (start 166 99) (end 166 100.03656) (width 0.25) (layer "F.Cu") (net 26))
 (segment (start 166 100.03656) (end 183.3 117.33656) (width 0.25) (layer "F.Cu") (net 26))
 (segment (start 162.96 95.96) (end 166 99) (width 0.25) (layer "F.Cu") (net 26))
 (segment (start 157.69 95.96) (end 162.96 95.96) (width 0.25) (layer "F.Cu") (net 26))
 (segment (start 113.69 117.96) (end 133.462613 117.96) (width 0.25) (layer "F.Cu") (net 27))
 (segment (start 138.562613 112.86) (end 171.20344 112.86) (width 0.25) (layer "F.Cu") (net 27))
 (segment (start 133.462613 117.96) (end 138.562613 112.86) (width 0.25) (layer "F.Cu") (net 27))
 (segment (start 171.20344 112.86) (end 183.3 124.95656) (width 0.25) (layer "F.Cu") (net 27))
 (segment (start 172.79844 116.995) (end 183.3 127.49656) (width 0.25) (layer "F.Cu") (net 10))
 (segment (start 145.04 117.96) (end 148 115) (width 0.25) (layer "F.Cu") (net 10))
 (segment (start 135.69 117.96) (end 145.04 117.96) (width 0.25) (layer "F.Cu") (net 10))
 (segment (start 161 115) (end 162.995 116.995) (width 0.25) (layer "F.Cu") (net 10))
 (segment (start 148 115) (end 161 115) (width 0.25) (layer "F.Cu") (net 10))
 (segment (start 162.995 116.995) (end 172.79844 116.995) (width 0.25) (layer "F.Cu") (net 10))
 (segment (start 183.3 130.03656) (end 180.03656 130.03656) (width 0.25) (layer "F.Cu") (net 28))
 (segment (start 180.03656 130.03656) (end 168 118) (width 0.25) (layer "F.Cu") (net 28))
 (segment (start 157.73 118) (end 157.69 117.96) (width 0.25) (layer "F.Cu") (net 28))
 (segment (start 168 118) (end 157.73 118) (width 0.25) (layer "F.Cu") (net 28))
 (segment (start 113.69 139.96) (end 121.07344 132.57656) (width 0.25) (layer "F.Cu") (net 29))
 (segment (start 121.07344 132.57656) (end 183.3 132.57656) (width 0.25) (layer "F.Cu") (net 29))
 (segment (start 203 110.33656) (end 208.7 104.63656) (width 0.25) (layer "F.Cu") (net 9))
 (segment (start 156 135) (end 181.708412 135) (width 0.25) (layer "F.Cu") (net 9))
 (segment (start 151.04 139.96) (end 156 135) (width 0.25) (layer "F.Cu") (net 9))
 (segment (start 203 114.584708) (end 203 110.33656) (width 0.25) (layer "F.Cu") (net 9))
 (segment (start 135.69 139.96) (end 151.04 139.96) (width 0.25) (layer "F.Cu") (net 9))
 (segment (start 181.708412 135) (end 182.516852 134.19156) (width 0.25) (layer "F.Cu") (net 9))
 (segment (start 183.393148 134.19156) (end 203 114.584708) (width 0.25) (layer "F.Cu") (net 9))
 (segment (start 182.516852 134.19156) (end 183.393148 134.19156) (width 0.25) (layer "F.Cu") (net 9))
 (segment (start 207.82344 107.17656) (end 208.7 107.17656) (width 0.25) (layer "F.Cu") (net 49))
 (segment (start 157.69 139.96) (end 176.748412 139.96) (width 0.25) (layer "F.Cu") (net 49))
 (segment (start 182.516852 136.04156) (end 184.45844 136.04156) (width 0.25) (layer "F.Cu") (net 49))
 (segment (start 182.475292 136) (end 182.516852 136.04156) (width 0.25) (layer "F.Cu") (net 49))
 (segment (start 176.748412 139.96) (end 180.708412 136) (width 0.25) (layer "F.Cu") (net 49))
 (segment (start 204 116.5) (end 204 111) (width 0.25) (layer "F.Cu") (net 49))
 (segment (start 180.708412 136) (end 182.475292 136) (width 0.25) (layer "F.Cu") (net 49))
 (segment (start 204 111) (end 207.82344 107.17656) (width 0.25) (layer "F.Cu") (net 49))
 (segment (start 184.45844 136.04156) (end 204 116.5) (width 0.25) (layer "F.Cu") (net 49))
 (segment (start 131.04 161.96) (end 138 155) (width 0.25) (layer "F.Cu") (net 46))
 (segment (start 187 151) (end 187 136) (width 0.25) (layer "F.Cu") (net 46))
 (segment (start 138 155) (end 183 155) (width 0.25) (layer "F.Cu") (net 46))
 (segment (start 187 136) (end 208.20344 114.79656) (width 0.25) (layer "F.Cu") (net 46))
 (segment (start 183 155) (end 187 151) (width 0.25) (layer "F.Cu") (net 46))
 (segment (start 208.20344 114.79656) (end 208.7 114.79656) (width 0.25) (layer "F.Cu") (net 46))
 (segment (start 113.69 161.96) (end 131.04 161.96) (width 0.25) (layer "F.Cu") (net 46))
 (segment (start 208.7 119.87656) (end 189 139.57656) (width 0.25) (layer "F.Cu") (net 17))
 (segment (start 140.65 157) (end 135.69 161.96) (width 0.25) (layer "F.Cu") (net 17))
 (segment (start 189 152) (end 184 157) (width 0.25) (layer "F.Cu") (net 17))
 (segment (start 189 139.57656) (end 189 152) (width 0.25) (layer "F.Cu") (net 17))
 (segment (start 184 157) (end 140.65 157) (width 0.25) (layer "F.Cu") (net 17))
 (segment (start 157.69 161.96) (end 182.04 161.96) (width 0.25) (layer "F.Cu") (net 44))
 (segment (start 191 140) (end 208.58344 122.41656) (width 0.25) (layer "F.Cu") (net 44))
 (segment (start 182.04 161.96) (end 191 153) (width 0.25) (layer "F.Cu") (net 44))
 (segment (start 208.58344 122.41656) (end 208.7 122.41656) (width 0.25) (layer "F.Cu") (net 44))
 (segment (start 191 153) (end 191 140) (width 0.25) (layer "F.Cu") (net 44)))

